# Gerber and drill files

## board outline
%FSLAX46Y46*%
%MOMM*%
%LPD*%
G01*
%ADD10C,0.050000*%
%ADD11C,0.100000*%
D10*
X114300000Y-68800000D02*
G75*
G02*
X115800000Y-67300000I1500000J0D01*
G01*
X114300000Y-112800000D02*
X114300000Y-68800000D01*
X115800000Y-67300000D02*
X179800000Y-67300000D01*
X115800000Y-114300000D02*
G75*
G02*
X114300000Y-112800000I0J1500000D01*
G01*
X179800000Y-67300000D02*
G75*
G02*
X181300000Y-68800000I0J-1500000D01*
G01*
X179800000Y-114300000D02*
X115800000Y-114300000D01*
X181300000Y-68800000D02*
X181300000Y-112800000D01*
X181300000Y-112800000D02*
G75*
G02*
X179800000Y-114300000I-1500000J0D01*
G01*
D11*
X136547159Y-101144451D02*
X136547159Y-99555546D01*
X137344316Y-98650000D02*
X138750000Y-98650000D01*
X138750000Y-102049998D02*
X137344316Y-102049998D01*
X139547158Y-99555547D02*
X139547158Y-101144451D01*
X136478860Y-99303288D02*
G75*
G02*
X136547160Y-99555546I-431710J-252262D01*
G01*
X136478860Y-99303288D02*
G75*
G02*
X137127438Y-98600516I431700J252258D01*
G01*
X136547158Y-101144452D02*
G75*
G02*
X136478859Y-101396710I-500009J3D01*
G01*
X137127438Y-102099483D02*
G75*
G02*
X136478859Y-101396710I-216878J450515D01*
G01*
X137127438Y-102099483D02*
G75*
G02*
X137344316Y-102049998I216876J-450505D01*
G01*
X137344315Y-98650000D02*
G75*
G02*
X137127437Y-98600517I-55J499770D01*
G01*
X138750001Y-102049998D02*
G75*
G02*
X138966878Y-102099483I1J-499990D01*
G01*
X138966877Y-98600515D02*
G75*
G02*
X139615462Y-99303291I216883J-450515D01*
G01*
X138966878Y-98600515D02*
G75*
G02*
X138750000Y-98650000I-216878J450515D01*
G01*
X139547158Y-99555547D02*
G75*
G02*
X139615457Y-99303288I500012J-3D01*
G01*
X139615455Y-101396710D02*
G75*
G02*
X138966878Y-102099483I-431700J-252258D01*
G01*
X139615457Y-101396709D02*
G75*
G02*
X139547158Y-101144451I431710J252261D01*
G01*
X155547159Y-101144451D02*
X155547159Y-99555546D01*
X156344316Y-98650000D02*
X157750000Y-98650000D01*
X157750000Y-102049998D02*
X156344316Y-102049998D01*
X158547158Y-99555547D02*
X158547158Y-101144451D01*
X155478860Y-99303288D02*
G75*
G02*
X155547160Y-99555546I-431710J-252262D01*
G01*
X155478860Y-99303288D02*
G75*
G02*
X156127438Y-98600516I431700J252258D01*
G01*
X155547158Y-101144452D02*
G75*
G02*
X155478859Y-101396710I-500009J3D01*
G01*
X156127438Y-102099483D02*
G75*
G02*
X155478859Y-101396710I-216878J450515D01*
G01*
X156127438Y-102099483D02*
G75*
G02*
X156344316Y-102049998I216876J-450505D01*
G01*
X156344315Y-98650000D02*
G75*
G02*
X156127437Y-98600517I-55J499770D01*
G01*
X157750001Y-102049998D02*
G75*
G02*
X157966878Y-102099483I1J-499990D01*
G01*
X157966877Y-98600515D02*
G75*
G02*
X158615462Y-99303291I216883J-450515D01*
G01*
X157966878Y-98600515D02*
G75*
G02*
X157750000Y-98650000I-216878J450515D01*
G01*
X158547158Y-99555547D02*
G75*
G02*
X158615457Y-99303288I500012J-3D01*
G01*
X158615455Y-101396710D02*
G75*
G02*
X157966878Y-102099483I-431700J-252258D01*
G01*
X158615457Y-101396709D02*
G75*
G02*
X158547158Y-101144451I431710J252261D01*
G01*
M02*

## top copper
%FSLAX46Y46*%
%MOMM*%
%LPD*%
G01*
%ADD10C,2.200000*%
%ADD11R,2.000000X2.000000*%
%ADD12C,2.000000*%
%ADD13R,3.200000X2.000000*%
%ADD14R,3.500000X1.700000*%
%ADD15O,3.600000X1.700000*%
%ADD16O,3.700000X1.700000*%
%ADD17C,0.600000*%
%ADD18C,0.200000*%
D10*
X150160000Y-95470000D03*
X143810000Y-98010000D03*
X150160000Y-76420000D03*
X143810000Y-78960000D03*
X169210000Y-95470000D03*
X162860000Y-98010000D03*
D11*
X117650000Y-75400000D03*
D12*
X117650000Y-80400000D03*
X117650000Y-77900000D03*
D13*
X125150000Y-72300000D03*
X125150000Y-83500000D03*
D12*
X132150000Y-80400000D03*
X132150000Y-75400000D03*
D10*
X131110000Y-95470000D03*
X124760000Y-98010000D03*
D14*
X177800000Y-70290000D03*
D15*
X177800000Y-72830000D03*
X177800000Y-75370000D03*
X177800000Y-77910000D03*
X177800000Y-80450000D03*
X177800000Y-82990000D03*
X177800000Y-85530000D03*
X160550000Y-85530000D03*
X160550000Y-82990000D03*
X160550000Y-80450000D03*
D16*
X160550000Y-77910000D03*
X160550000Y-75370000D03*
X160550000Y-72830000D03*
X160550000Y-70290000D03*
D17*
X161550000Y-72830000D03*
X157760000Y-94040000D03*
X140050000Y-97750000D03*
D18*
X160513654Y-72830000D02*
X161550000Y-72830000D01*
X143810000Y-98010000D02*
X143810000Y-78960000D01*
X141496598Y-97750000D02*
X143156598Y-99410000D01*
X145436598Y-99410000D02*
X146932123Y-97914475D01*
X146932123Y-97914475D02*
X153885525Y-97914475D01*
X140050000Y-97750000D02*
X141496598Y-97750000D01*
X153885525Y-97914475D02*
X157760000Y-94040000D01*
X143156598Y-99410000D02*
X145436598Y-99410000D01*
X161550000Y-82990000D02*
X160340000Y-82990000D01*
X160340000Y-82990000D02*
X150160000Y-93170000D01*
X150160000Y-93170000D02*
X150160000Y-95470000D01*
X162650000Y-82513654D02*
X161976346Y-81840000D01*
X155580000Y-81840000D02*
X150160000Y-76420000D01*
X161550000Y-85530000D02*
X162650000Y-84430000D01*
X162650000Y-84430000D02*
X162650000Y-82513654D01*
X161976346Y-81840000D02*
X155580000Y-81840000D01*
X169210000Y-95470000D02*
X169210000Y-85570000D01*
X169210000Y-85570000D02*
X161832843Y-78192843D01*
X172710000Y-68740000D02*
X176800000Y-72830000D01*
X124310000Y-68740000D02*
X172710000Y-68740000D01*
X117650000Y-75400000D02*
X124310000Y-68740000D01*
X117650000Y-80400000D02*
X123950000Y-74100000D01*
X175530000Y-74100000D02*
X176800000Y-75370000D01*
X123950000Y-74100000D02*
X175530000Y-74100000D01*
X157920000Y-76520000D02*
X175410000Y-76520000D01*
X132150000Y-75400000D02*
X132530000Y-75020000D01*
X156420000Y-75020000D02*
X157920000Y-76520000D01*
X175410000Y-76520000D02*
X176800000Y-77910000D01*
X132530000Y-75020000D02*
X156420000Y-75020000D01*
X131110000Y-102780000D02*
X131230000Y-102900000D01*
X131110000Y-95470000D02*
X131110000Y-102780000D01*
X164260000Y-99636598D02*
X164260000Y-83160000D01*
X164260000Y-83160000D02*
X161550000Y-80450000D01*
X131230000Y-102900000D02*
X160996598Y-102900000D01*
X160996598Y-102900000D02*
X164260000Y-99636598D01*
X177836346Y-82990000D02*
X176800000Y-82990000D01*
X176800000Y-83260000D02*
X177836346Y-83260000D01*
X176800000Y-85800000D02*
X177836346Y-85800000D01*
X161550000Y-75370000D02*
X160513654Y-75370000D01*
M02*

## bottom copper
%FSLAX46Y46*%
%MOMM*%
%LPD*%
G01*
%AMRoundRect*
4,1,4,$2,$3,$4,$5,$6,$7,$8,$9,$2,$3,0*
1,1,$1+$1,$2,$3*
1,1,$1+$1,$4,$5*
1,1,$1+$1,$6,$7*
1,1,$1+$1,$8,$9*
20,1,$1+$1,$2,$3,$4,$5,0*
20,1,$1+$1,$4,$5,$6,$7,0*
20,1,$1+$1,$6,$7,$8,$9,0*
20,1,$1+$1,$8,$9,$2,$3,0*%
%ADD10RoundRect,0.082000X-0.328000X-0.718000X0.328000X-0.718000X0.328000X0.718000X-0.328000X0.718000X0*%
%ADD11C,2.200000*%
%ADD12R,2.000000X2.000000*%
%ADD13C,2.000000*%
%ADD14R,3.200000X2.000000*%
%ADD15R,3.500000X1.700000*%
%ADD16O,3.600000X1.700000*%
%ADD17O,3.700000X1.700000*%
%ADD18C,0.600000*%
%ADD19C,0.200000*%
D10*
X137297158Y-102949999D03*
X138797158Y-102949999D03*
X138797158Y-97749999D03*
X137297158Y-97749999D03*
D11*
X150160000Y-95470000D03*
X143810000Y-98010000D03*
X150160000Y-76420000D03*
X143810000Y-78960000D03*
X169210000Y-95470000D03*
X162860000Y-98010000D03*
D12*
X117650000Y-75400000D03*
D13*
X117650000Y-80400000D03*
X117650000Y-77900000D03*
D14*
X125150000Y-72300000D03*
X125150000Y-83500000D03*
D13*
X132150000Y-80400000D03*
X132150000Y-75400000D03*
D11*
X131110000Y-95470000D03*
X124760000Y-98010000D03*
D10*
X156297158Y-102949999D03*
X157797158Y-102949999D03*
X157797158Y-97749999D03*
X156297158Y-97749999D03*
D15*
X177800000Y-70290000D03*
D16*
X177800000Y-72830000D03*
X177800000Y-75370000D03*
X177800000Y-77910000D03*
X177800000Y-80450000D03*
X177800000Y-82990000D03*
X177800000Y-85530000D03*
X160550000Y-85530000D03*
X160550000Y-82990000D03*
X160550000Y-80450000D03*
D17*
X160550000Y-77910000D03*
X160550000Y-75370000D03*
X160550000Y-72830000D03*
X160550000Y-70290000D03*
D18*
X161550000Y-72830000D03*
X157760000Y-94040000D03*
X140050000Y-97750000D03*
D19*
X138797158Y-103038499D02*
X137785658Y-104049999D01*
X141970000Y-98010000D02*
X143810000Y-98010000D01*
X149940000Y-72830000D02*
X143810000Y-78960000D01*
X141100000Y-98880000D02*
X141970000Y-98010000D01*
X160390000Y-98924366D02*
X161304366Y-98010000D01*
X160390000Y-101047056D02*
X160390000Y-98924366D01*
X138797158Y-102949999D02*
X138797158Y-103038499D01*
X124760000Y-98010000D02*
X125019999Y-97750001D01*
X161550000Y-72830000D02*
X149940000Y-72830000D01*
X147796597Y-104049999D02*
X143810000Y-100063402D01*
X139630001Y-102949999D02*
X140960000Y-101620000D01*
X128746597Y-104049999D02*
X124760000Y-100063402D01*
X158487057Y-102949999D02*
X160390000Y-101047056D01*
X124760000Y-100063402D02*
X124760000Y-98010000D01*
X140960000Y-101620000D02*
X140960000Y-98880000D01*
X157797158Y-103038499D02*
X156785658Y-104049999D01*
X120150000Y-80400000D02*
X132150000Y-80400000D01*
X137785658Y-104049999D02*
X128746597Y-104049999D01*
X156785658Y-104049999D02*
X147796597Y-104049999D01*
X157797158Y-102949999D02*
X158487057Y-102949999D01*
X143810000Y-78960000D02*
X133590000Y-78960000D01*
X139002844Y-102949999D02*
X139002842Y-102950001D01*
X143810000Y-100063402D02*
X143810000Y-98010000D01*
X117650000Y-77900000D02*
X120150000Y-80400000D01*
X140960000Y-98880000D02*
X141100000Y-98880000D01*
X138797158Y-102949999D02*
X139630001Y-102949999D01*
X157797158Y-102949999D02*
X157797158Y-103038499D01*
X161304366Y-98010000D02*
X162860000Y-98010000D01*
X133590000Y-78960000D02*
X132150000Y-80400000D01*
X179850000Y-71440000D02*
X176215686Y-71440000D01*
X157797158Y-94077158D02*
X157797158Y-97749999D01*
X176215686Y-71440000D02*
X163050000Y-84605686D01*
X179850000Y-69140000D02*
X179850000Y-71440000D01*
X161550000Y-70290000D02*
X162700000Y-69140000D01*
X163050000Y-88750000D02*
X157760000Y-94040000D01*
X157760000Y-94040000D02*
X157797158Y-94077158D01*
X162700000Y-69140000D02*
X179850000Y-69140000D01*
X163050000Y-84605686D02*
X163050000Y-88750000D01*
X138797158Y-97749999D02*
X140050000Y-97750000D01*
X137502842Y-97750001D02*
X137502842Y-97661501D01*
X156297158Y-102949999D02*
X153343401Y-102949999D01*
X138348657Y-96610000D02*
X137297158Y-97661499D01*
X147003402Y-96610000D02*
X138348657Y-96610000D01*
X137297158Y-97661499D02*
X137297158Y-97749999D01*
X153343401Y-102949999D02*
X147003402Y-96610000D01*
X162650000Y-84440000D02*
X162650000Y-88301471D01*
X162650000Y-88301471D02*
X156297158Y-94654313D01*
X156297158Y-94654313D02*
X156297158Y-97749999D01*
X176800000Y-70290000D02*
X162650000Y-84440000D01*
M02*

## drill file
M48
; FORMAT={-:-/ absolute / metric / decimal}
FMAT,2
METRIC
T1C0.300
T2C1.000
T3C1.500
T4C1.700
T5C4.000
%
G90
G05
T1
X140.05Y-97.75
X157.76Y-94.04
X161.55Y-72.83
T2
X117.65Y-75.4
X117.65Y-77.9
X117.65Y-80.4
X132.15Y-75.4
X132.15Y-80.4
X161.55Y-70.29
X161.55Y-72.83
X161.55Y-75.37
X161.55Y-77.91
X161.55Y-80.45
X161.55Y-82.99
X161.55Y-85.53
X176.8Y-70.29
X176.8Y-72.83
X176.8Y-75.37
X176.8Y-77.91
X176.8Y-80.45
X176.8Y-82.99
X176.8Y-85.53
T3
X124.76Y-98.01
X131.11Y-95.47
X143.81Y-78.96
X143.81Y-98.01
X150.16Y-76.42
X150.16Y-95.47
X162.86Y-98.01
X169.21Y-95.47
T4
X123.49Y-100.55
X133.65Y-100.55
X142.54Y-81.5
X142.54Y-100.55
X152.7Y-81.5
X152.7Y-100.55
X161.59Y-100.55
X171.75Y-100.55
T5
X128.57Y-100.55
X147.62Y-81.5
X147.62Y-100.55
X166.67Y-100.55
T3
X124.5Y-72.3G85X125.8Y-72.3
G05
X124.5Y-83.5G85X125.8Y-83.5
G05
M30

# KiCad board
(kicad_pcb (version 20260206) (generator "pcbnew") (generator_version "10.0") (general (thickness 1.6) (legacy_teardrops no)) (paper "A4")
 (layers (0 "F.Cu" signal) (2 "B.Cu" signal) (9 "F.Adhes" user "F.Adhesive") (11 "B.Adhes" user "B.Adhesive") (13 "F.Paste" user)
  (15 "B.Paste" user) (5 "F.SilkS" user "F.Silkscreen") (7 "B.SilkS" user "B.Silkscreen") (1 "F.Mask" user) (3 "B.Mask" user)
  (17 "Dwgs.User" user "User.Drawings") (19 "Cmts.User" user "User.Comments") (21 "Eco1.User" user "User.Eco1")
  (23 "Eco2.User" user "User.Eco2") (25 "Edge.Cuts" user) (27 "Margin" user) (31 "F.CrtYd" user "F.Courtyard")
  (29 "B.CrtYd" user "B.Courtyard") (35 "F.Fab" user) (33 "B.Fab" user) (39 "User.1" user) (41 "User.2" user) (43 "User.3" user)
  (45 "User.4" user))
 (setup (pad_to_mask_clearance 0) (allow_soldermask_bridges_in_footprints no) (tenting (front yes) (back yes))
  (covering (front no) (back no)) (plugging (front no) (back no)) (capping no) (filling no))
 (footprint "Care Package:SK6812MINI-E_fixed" (layer "F.Cu") (at 138.15 100.35 90)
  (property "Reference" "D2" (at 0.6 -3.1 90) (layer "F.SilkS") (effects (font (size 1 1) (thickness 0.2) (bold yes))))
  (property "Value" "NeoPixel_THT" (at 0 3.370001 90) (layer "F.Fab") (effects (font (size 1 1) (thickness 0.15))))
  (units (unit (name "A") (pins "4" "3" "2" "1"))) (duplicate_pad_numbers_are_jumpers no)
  (fp_line (start -0.794451 -1.602841) (end 0.794454 -1.602841) (stroke (width 0.1) (type solid)) (layer "Edge.Cuts"))
  (fp_line (start 1.7 -0.805684) (end 1.7 0.6) (stroke (width 0.1) (type solid)) (layer "Edge.Cuts"))
  (fp_line (start -1.699998 0.6) (end -1.699998 -0.805684) (stroke (width 0.1) (type solid)) (layer "Edge.Cuts"))
  (fp_line (start 0.794453 1.397158) (end -0.794451 1.397158) (stroke (width 0.1) (type solid)) (layer "Edge.Cuts"))
  (fp_arc (start 1.046712 -1.67114) (mid 0.925124 -1.620218) (end 0.794454 -1.602841) (stroke (width 0.1) (type solid)) (layer "Edge.Cuts"))
  (fp_arc (start 1.046712 -1.67114) (mid 1.638071 -1.606876) (end 1.749485 -1.022562) (stroke (width 0.1) (type solid)) (layer "Edge.Cuts"))
  (fp_arc (start -0.794452 -1.602842) (mid -0.925122 -1.620219) (end -1.04671 -1.671141) (stroke (width 0.1) (type solid))
   (layer "Edge.Cuts"))
  (fp_arc (start -1.749483 -1.022562) (mid -1.63807 -1.606877) (end -1.04671 -1.671141) (stroke (width 0.1) (type solid))
   (layer "Edge.Cuts"))
  (fp_arc (start -1.749483 -1.022562) (mid -1.712526 -0.91691) (end -1.699998 -0.805684) (stroke (width 0.1) (type solid))
   (layer "Edge.Cuts"))
  (fp_arc (start 1.7 -0.805685) (mid 1.712523 -0.916913) (end 1.749485 -1.022562) (stroke (width 0.1) (type solid)) (layer "Edge.Cuts"))
  (fp_arc (start -1.699998 0.600001) (mid -1.712526 0.711226) (end -1.749483 0.816878) (stroke (width 0.1) (type solid)) (layer "Edge.Cuts"))
  (fp_arc (start 1.749485 0.816877) (mid 1.638074 1.401197) (end 1.046712 1.465457) (stroke (width 0.1) (type solid)) (layer "Edge.Cuts"))
  (fp_arc (start 1.749485 0.816878) (mid 1.712528 0.711226) (end 1.7 0.6) (stroke (width 0.1) (type solid)) (layer "Edge.Cuts"))
  (fp_arc (start 0.794453 1.397158) (mid 0.925124 1.414535) (end 1.046712 1.465457) (stroke (width 0.1) (type solid)) (layer "Edge.Cuts"))
  (fp_arc (start -1.04671 1.465455) (mid -1.638069 1.401192) (end -1.749483 0.816878) (stroke (width 0.1) (type solid)) (layer "Edge.Cuts"))
  (fp_arc (start -1.046709 1.465457) (mid -0.925121 1.414535) (end -0.794451 1.397158) (stroke (width 0.1) (type solid)) (layer "Edge.Cuts"))
  (pad "1" smd roundrect (at -2.599999 -0.852842) (size 0.82 1.6) (layers "B.Cu" "B.Mask" "B.Paste") (roundrect_rratio 0.1)
   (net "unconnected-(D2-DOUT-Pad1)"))
  (pad "2" smd roundrect (at -2.599999 0.647158) (size 0.82 1.6) (layers "B.Cu" "B.Mask" "B.Paste") (roundrect_rratio 0.1) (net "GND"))
  (pad "3" smd roundrect (at 2.600001 0.647158) (size 0.82 1.6) (layers "B.Cu" "B.Mask" "B.Paste") (roundrect_rratio 0.1) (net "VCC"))
  (pad "4" smd roundrect (at 2.600001 -0.852842) (size 0.82 1.6) (layers "B.Cu" "B.Mask" "B.Paste") (roundrect_rratio 0.1)
   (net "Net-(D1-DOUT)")))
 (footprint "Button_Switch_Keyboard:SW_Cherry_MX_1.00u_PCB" (layer "F.Cu") (at 150.16 95.47)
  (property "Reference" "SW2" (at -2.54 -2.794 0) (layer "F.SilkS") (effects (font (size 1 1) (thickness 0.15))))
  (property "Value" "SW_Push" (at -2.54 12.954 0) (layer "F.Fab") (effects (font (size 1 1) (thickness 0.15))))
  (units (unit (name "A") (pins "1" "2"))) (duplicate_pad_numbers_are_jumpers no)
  (pad "" np_thru_hole circle (at -7.62 5.08) (size 1.7 1.7) (drill 1.7) (layers "*.Cu" "*.Mask"))
  (pad "" np_thru_hole circle (at -2.54 5.08) (size 4 4) (drill 4) (layers "*.Cu" "*.Mask"))
  (pad "" np_thru_hole circle (at 2.54 5.08) (size 1.7 1.7) (drill 1.7) (layers "*.Cu" "*.Mask"))
  (pad "1" thru_hole circle (at 0 0) (size 2.2 2.2) (drill 1.5) (layers "*.Cu" "*.Mask") (remove_unused_layers no)
   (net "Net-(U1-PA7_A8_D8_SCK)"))
  (pad "2" thru_hole circle (at -6.35 2.54) (size 2.2 2.2) (drill 1.5) (layers "*.Cu" "*.Mask") (remove_unused_layers no) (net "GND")))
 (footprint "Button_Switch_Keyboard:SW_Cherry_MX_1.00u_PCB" (layer "F.Cu") (at 150.16 76.42)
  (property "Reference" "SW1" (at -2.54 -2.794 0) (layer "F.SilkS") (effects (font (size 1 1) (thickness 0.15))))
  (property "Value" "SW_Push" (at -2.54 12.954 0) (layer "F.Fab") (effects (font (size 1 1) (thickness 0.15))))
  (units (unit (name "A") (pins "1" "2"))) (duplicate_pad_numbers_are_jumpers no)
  (pad "" np_thru_hole circle (at -7.62 5.08) (size 1.7 1.7) (drill 1.7) (layers "*.Cu" "*.Mask"))
  (pad "" np_thru_hole circle (at -2.54 5.08) (size 4 4) (drill 4) (layers "*.Cu" "*.Mask"))
  (pad "" np_thru_hole circle (at 2.54 5.08) (size 1.7 1.7) (drill 1.7) (layers "*.Cu" "*.Mask"))
  (pad "1" thru_hole circle (at 0 0) (size 2.2 2.2) (drill 1.5) (layers "*.Cu" "*.Mask") (remove_unused_layers no)
   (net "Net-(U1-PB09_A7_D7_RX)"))
  (pad "2" thru_hole circle (at -6.35 2.54) (size 2.2 2.2) (drill 1.5) (layers "*.Cu" "*.Mask") (remove_unused_layers no) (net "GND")))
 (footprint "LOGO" (layer "F.Cu") (at 176.41 109.06)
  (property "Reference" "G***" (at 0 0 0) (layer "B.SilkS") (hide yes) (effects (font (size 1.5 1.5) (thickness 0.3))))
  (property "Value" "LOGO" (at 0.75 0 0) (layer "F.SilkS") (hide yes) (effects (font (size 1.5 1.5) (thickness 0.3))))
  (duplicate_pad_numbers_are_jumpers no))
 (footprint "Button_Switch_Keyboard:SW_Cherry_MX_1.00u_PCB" (layer "F.Cu") (at 169.21 95.47)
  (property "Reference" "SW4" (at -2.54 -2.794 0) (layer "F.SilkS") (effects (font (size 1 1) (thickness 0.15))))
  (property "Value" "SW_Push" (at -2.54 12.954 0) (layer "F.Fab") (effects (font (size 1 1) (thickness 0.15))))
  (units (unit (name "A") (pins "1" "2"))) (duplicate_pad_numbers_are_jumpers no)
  (pad "" np_thru_hole circle (at -7.62 5.08) (size 1.7 1.7) (drill 1.7) (layers "*.Cu" "*.Mask"))
  (pad "" np_thru_hole circle (at -2.54 5.08) (size 4 4) (drill 4) (layers "*.Cu" "*.Mask"))
  (pad "" np_thru_hole circle (at 2.54 5.08) (size 1.7 1.7) (drill 1.7) (layers "*.Cu" "*.Mask"))
  (pad "1" thru_hole circle (at 0 0) (size 2.2 2.2) (drill 1.5) (layers "*.Cu" "*.Mask") (remove_unused_layers no)
   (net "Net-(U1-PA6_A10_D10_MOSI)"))
  (pad "2" thru_hole circle (at -6.35 2.54) (size 2.2 2.2) (drill 1.5) (layers "*.Cu" "*.Mask") (remove_unused_layers no) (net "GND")))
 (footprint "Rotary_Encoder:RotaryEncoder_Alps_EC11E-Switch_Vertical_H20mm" (layer "F.Cu") (at 117.65 75.4)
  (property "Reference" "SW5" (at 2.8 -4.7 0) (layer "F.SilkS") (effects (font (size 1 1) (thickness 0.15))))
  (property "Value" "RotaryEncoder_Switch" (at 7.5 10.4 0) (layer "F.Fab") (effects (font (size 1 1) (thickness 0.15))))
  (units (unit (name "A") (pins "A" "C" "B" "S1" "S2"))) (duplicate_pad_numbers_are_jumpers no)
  (pad "A" thru_hole rect (at 0 0) (size 2 2) (drill 1) (layers "*.Cu" "*.Mask") (remove_unused_layers no) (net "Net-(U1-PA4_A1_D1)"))
  (pad "B" thru_hole circle (at 0 5) (size 2 2) (drill 1) (layers "*.Cu" "*.Mask") (remove_unused_layers no) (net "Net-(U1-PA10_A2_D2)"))
  (pad "C" thru_hole circle (at 0 2.5) (size 2 2) (drill 1) (layers "*.Cu" "*.Mask") (remove_unused_layers no) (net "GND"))
  (pad "MP" thru_hole rect (at 7.5 -3.1) (size 3.2 2) (drill oval 2.8 1.5) (layers "*.Cu" "*.Mask") (remove_unused_layers no))
  (pad "MP" thru_hole rect (at 7.5 8.1) (size 3.2 2) (drill oval 2.8 1.5) (layers "*.Cu" "*.Mask") (remove_unused_layers no))
  (pad "S1" thru_hole circle (at 14.5 5) (size 2 2) (drill 1) (layers "*.Cu" "*.Mask") (remove_unused_layers no) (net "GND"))
  (pad "S2" thru_hole circle (at 14.5 0) (size 2 2) (drill 1) (layers "*.Cu" "*.Mask") (remove_unused_layers no) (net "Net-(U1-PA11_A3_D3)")))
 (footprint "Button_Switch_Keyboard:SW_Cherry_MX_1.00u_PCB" (layer "F.Cu") (at 131.11 95.47)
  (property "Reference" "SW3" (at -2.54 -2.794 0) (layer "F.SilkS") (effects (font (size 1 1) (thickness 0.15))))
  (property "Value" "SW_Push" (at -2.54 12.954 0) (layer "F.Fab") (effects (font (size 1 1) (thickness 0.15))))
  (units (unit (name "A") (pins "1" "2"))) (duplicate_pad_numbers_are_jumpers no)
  (pad "" np_thru_hole circle (at -7.62 5.08) (size 1.7 1.7) (drill 1.7) (layers "*.Cu" "*.Mask"))
  (pad "" np_thru_hole circle (at -2.54 5.08) (size 4 4) (drill 4) (layers "*.Cu" "*.Mask"))
  (pad "" np_thru_hole circle (at 2.54 5.08) (size 1.7 1.7) (drill 1.7) (layers "*.Cu" "*.Mask"))
  (pad "1" thru_hole circle (at 0 0) (size 2.2 2.2) (drill 1.5) (layers "*.Cu" "*.Mask") (remove_unused_layers no)
   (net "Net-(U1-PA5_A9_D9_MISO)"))
  (pad "2" thru_hole circle (at -6.35 2.54) (size 2.2 2.2) (drill 1.5) (layers "*.Cu" "*.Mask") (remove_unused_layers no) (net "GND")))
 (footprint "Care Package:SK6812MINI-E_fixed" (layer "F.Cu") (at 157.15 100.35 90)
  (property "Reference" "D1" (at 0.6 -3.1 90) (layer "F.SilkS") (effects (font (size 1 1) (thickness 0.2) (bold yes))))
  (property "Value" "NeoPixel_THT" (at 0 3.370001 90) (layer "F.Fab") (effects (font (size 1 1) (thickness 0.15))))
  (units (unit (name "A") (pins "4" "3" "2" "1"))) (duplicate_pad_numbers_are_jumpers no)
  (fp_line (start -0.794451 -1.602841) (end 0.794454 -1.602841) (stroke (width 0.1) (type solid)) (layer "Edge.Cuts"))
  (fp_line (start 1.7 -0.805684) (end 1.7 0.6) (stroke (width 0.1) (type solid)) (layer "Edge.Cuts"))
  (fp_line (start -1.699998 0.6) (end -1.699998 -0.805684) (stroke (width 0.1) (type solid)) (layer "Edge.Cuts"))
  (fp_line (start 0.794453 1.397158) (end -0.794451 1.397158) (stroke (width 0.1) (type solid)) (layer "Edge.Cuts"))
  (fp_arc (start 1.046712 -1.67114) (mid 0.925124 -1.620218) (end 0.794454 -1.602841) (stroke (width 0.1) (type solid)) (layer "Edge.Cuts"))
  (fp_arc (start 1.046712 -1.67114) (mid 1.638071 -1.606876) (end 1.749485 -1.022562) (stroke (width 0.1) (type solid)) (layer "Edge.Cuts"))
  (fp_arc (start -0.794452 -1.602842) (mid -0.925122 -1.620219) (end -1.04671 -1.671141) (stroke (width 0.1) (type solid))
   (layer "Edge.Cuts"))
  (fp_arc (start -1.749483 -1.022562) (mid -1.63807 -1.606877) (end -1.04671 -1.671141) (stroke (width 0.1) (type solid))
   (layer "Edge.Cuts"))
  (fp_arc (start -1.749483 -1.022562) (mid -1.712526 -0.91691) (end -1.699998 -0.805684) (stroke (width 0.1) (type solid))
   (layer "Edge.Cuts"))
  (fp_arc (start 1.7 -0.805685) (mid 1.712523 -0.916913) (end 1.749485 -1.022562) (stroke (width 0.1) (type solid)) (layer "Edge.Cuts"))
  (fp_arc (start -1.699998 0.600001) (mid -1.712526 0.711226) (end -1.749483 0.816878) (stroke (width 0.1) (type solid)) (layer "Edge.Cuts"))
  (fp_arc (start 1.749485 0.816877) (mid 1.638074 1.401197) (end 1.046712 1.465457) (stroke (width 0.1) (type solid)) (layer "Edge.Cuts"))
  (fp_arc (start 1.749485 0.816878) (mid 1.712528 0.711226) (end 1.7 0.6) (stroke (width 0.1) (type solid)) (layer "Edge.Cuts"))
  (fp_arc (start 0.794453 1.397158) (mid 0.925124 1.414535) (end 1.046712 1.465457) (stroke (width 0.1) (type solid)) (layer "Edge.Cuts"))
  (fp_arc (start -1.04671 1.465455) (mid -1.638069 1.401192) (end -1.749483 0.816878) (stroke (width 0.1) (type solid)) (layer "Edge.Cuts"))
  (fp_arc (start -1.046709 1.465457) (mid -0.925121 1.414535) (end -0.794451 1.397158) (stroke (width 0.1) (type solid)) (layer "Edge.Cuts"))
  (pad "1" smd roundrect (at -2.599999 -0.852842) (size 0.82 1.6) (layers "B.Cu" "B.Mask" "B.Paste") (roundrect_rratio 0.1)
   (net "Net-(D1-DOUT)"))
  (pad "2" smd roundrect (at -2.599999 0.647158) (size 0.82 1.6) (layers "B.Cu" "B.Mask" "B.Paste") (roundrect_rratio 0.1) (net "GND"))
  (pad "3" smd roundrect (at 2.600001 0.647158) (size 0.82 1.6) (layers "B.Cu" "B.Mask" "B.Paste") (roundrect_rratio 0.1) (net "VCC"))
  (pad "4" smd roundrect (at 2.600001 -0.852842) (size 0.82 1.6) (layers "B.Cu" "B.Mask" "B.Paste") (roundrect_rratio 0.1)
   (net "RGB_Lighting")))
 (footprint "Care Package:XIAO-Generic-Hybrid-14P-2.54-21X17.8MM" (layer "B.Cu") (at 169.175 77.91 180)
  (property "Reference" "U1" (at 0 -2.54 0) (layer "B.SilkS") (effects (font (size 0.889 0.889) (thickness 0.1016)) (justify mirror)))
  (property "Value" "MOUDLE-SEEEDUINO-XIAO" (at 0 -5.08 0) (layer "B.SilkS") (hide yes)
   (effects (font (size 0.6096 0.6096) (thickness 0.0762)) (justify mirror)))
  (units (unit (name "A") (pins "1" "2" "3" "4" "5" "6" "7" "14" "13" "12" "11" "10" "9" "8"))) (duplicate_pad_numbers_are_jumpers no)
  (pad "1" thru_hole rect (at -7.625 7.62 180) (size 3.5 1.7) (drill 1 (offset -1 0)) (layers "*.Cu" "*.Mask") (remove_unused_layers no)
   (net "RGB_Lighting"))
  (pad "2" thru_hole oval (at -7.625 5.08 180) (size 3.6 1.7) (drill 1 (offset -1 0)) (layers "*.Cu" "*.Mask") (remove_unused_layers no)
   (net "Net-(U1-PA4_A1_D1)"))
  (pad "3" thru_hole oval (at -7.625 2.54 180) (size 3.6 1.7) (drill 1 (offset -1 0)) (layers "*.Cu" "*.Mask") (remove_unused_layers no)
   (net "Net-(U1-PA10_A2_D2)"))
  (pad "4" thru_hole oval (at -7.625 0 180) (size 3.6 1.7) (drill 1 (offset -1 0)) (layers "*.Cu" "*.Mask") (remove_unused_layers no)
   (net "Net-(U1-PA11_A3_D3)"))
  (pad "5" thru_hole oval (at -7.625 -2.54 180) (size 3.6 1.7) (drill 1 (offset -1 0)) (layers "*.Cu" "*.Mask") (remove_unused_layers no)
   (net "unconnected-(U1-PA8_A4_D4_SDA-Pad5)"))
  (pad "6" thru_hole oval (at -7.625 -5.08) (size 3.6 1.7) (drill 1 (offset 1 0)) (layers "*.Cu" "*.Mask") (remove_unused_layers no)
   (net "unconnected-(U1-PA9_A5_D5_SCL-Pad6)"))
  (pad "7" thru_hole oval (at -7.625 -7.62 180) (size 3.6 1.7) (drill 1 (offset -1 0)) (layers "*.Cu" "*.Mask") (remove_unused_layers no)
   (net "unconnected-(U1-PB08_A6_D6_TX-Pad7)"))
  (pad "8" thru_hole oval (at 7.625 -7.62 180) (size 3.6 1.7) (drill 1 (offset 1 0)) (layers "*.Cu" "*.Mask") (remove_unused_layers no)
   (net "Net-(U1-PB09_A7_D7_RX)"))
  (pad "9" thru_hole oval (at 7.625 -5.08 180) (size 3.6 1.7) (drill 1 (offset 1 0)) (layers "*.Cu" "*.Mask") (remove_unused_layers no)
   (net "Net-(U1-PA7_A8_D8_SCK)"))
  (pad "10" thru_hole oval (at 7.625 -2.54 180) (size 3.6 1.7) (drill 1 (offset 1 0)) (layers "*.Cu" "*.Mask") (remove_unused_layers no)
   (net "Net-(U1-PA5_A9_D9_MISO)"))
  (pad "11" thru_hole oval (at 7.625 0 180) (size 3.7 1.7) (drill 1 (offset 1 0)) (layers "*.Cu" "*.Mask") (remove_unused_layers no)
   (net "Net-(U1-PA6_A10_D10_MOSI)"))
  (pad "12" thru_hole oval (at 7.625 2.54 180) (size 3.7 1.7) (drill 1 (offset 1 0)) (layers "*.Cu" "*.Mask") (remove_unused_layers no)
   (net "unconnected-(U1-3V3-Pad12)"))
  (pad "13" thru_hole oval (at 7.625 5.08 180) (size 3.7 1.7) (drill 1 (offset 1 0)) (layers "*.Cu" "*.Mask") (remove_unused_layers no)
   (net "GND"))
  (pad "14" thru_hole oval (at 7.625 7.62 180) (size 3.7 1.7) (drill 1 (offset 1 0)) (layers "*.Cu" "*.Mask") (remove_unused_layers no)
   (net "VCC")))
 (gr_arc (start 114.3 68.8) (mid 114.73934 67.73934) (end 115.8 67.3) (stroke (width 0.05) (type default)) (layer "Edge.Cuts"))
 (gr_line (start 114.3 112.8) (end 114.3 68.8) (stroke (width 0.05) (type default)) (layer "Edge.Cuts"))
 (gr_line (start 115.8 67.3) (end 179.8 67.3) (stroke (width 0.05) (type default)) (layer "Edge.Cuts"))
 (gr_arc (start 115.8 114.3) (mid 114.73934 113.86066) (end 114.3 112.8) (stroke (width 0.05) (type default)) (layer "Edge.Cuts"))
 (gr_arc (start 179.8 67.3) (mid 180.86066 67.73934) (end 181.3 68.8) (stroke (width 0.05) (type default)) (layer "Edge.Cuts"))
 (gr_line (start 179.8 114.3) (end 115.8 114.3) (stroke (width 0.05) (type default)) (layer "Edge.Cuts"))
 (gr_line (start 181.3 68.8) (end 181.3 112.8) (stroke (width 0.05) (type default)) (layer "Edge.Cuts"))
 (gr_arc (start 181.3 112.8) (mid 180.86066 113.86066) (end 179.8 114.3) (stroke (width 0.05) (type default)) (layer "Edge.Cuts"))
 (segment (start 160.513654 72.83) (end 161.55 72.83) (width 0.2) (layer "F.Cu") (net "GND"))
 (segment (start 143.81 98.01) (end 143.81 78.96) (width 0.2) (layer "F.Cu") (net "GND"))
 (via (at 161.55 72.83) (size 0.6) (drill 0.3) (layers "F.Cu" "B.Cu") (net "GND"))
 (segment (start 138.797158 103.038499) (end 137.785658 104.049999) (width 0.2) (layer "B.Cu") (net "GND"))
 (segment (start 141.97 98.01) (end 143.81 98.01) (width 0.2) (layer "B.Cu") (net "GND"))
 (segment (start 149.94 72.83) (end 143.81 78.96) (width 0.2) (layer "B.Cu") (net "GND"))
 (segment (start 141.1 98.88) (end 141.97 98.01) (width 0.2) (layer "B.Cu") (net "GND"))
 (segment (start 160.39 98.924366) (end 161.304366 98.01) (width 0.2) (layer "B.Cu") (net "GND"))
 (segment (start 160.39 101.047056) (end 160.39 98.924366) (width 0.2) (layer "B.Cu") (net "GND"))
 (segment (start 138.797158 102.949999) (end 138.797158 103.038499) (width 0.2) (layer "B.Cu") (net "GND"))
 (segment (start 124.76 98.01) (end 125.019999 97.750001) (width 0.2) (layer "B.Cu") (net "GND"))
 (segment (start 161.55 72.83) (end 149.94 72.83) (width 0.2) (layer "B.Cu") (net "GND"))
 (segment (start 147.796597 104.049999) (end 143.81 100.063402) (width 0.2) (layer "B.Cu") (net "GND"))
 (segment (start 139.630001 102.949999) (end 140.96 101.62) (width 0.2) (layer "B.Cu") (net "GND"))
 (segment (start 128.746597 104.049999) (end 124.76 100.063402) (width 0.2) (layer "B.Cu") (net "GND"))
 (segment (start 158.487057 102.949999) (end 160.39 101.047056) (width 0.2) (layer "B.Cu") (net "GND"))
 (segment (start 124.76 100.063402) (end 124.76 98.01) (width 0.2) (layer "B.Cu") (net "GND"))
 (segment (start 140.96 101.62) (end 140.96 98.88) (width 0.2) (layer "B.Cu") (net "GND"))
 (segment (start 157.797158 103.038499) (end 156.785658 104.049999) (width 0.2) (layer "B.Cu") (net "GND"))
 (segment (start 120.15 80.4) (end 132.15 80.4) (width 0.2) (layer "B.Cu") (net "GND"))
 (segment (start 137.785658 104.049999) (end 128.746597 104.049999) (width 0.2) (layer "B.Cu") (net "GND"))
 (segment (start 156.785658 104.049999) (end 147.796597 104.049999) (width 0.2) (layer "B.Cu") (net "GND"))
 (segment (start 157.797158 102.949999) (end 158.487057 102.949999) (width 0.2) (layer "B.Cu") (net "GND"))
 (segment (start 143.81 78.96) (end 133.59 78.96) (width 0.2) (layer "B.Cu") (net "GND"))
 (segment (start 139.002844 102.949999) (end 139.002842 102.950001) (width 0.2) (layer "B.Cu") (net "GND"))
 (segment (start 143.81 100.063402) (end 143.81 98.01) (width 0.2) (layer "B.Cu") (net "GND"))
 (segment (start 117.65 77.9) (end 120.15 80.4) (width 0.2) (layer "B.Cu") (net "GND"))
 (segment (start 140.96 98.88) (end 141.1 98.88) (width 0.2) (layer "B.Cu") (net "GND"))
 (segment (start 138.797158 102.949999) (end 139.630001 102.949999) (width 0.2) (layer "B.Cu") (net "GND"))
 (segment (start 157.797158 102.949999) (end 157.797158 103.038499) (width 0.2) (layer "B.Cu") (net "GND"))
 (segment (start 161.304366 98.01) (end 162.86 98.01) (width 0.2) (layer "B.Cu") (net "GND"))
 (segment (start 133.59 78.96) (end 132.15 80.4) (width 0.2) (layer "B.Cu") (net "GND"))
 (segment (start 141.496598 97.75) (end 143.156598 99.41) (width 0.2) (layer "F.Cu") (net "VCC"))
 (segment (start 145.436598 99.41) (end 146.932123 97.914475) (width 0.2) (layer "F.Cu") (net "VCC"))
 (segment (start 146.932123 97.914475) (end 153.885525 97.914475) (width 0.2) (layer "F.Cu") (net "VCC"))
 (segment (start 140.05 97.75) (end 141.496598 97.75) (width 0.2) (layer "F.Cu") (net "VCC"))
 (segment (start 153.885525 97.914475) (end 157.76 94.04) (width 0.2) (layer "F.Cu") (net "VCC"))
 (segment (start 143.156598 99.41) (end 145.436598 99.41) (width 0.2) (layer "F.Cu") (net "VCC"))
 (via (at 157.76 94.04) (size 0.6) (drill 0.3) (layers "F.Cu" "B.Cu") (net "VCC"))
 (via (at 140.05 97.75) (size 0.6) (drill 0.3) (layers "F.Cu" "B.Cu") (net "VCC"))
 (segment (start 179.85 71.44) (end 176.215686 71.44) (width 0.2) (layer "B.Cu") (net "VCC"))
 (segment (start 157.797158 94.077158) (end 157.797158 97.749999) (width 0.2) (layer "B.Cu") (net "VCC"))
 (segment (start 176.215686 71.44) (end 163.05 84.605686) (width 0.2) (layer "B.Cu") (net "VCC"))
 (segment (start 179.85 69.14) (end 179.85 71.44) (width 0.2) (layer "B.Cu") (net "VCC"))
 (segment (start 161.55 70.29) (end 162.7 69.14) (width 0.2) (layer "B.Cu") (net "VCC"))
 (segment (start 163.05 88.75) (end 157.76 94.04) (width 0.2) (layer "B.Cu") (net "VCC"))
 (segment (start 157.76 94.04) (end 157.797158 94.077158) (width 0.2) (layer "B.Cu") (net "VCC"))
 (segment (start 162.7 69.14) (end 179.85 69.14) (width 0.2) (layer "B.Cu") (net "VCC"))
 (segment (start 163.05 84.605686) (end 163.05 88.75) (width 0.2) (layer "B.Cu") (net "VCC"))
 (segment (start 138.797158 97.749999) (end 140.05 97.75) (width 0.2) (layer "B.Cu") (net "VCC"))
 (segment (start 137.502842 97.750001) (end 137.502842 97.661501) (width 0.2) (layer "B.Cu") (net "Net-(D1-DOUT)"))
 (segment (start 156.297158 102.949999) (end 153.343401 102.949999) (width 0.2) (layer "B.Cu") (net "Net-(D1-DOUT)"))
 (segment (start 138.348657 96.61) (end 137.297158 97.661499) (width 0.2) (layer "B.Cu") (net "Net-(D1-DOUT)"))
 (segment (start 147.003402 96.61) (end 138.348657 96.61) (width 0.2) (layer "B.Cu") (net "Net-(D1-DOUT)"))
 (segment (start 137.297158 97.661499) (end 137.297158 97.749999) (width 0.2) (layer "B.Cu") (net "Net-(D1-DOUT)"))
 (segment (start 153.343401 102.949999) (end 147.003402 96.61) (width 0.2) (layer "B.Cu") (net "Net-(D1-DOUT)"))
 (segment (start 161.55 82.99) (end 160.34 82.99) (width 0.2) (layer "F.Cu") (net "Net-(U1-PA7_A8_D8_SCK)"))
 (segment (start 160.34 82.99) (end 150.16 93.17) (width 0.2) (layer "F.Cu") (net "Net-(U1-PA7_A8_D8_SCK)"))
 (segment (start 150.16 93.17) (end 150.16 95.47) (width 0.2) (layer "F.Cu") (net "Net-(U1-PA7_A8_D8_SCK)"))
 (segment (start 162.65 82.513654) (end 161.976346 81.84) (width 0.2) (layer "F.Cu") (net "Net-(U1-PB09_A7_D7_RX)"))
 (segment (start 155.58 81.84) (end 150.16 76.42) (width 0.2) (layer "F.Cu") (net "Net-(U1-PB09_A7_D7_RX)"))
 (segment (start 161.55 85.53) (end 162.65 84.43) (width 0.2) (layer "F.Cu") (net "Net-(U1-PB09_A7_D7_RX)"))
 (segment (start 162.65 84.43) (end 162.65 82.513654) (width 0.2) (layer "F.Cu") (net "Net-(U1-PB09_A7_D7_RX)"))
 (segment (start 161.976346 81.84) (end 155.58 81.84) (width 0.2) (layer "F.Cu") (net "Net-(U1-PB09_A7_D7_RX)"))
 (segment (start 169.21 95.47) (end 169.21 85.57) (width 0.2) (layer "F.Cu") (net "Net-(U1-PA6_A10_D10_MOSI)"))
 (segment (start 169.21 85.57) (end 161.832843 78.192843) (width 0.2) (layer "F.Cu") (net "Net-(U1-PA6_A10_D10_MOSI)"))
 (segment (start 172.71 68.74) (end 176.8 72.83) (width 0.2) (layer "F.Cu") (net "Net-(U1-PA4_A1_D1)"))
 (segment (start 124.31 68.74) (end 172.71 68.74) (width 0.2) (layer "F.Cu") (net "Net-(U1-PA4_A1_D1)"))
 (segment (start 117.65 75.4) (end 124.31 68.74) (width 0.2) (layer "F.Cu") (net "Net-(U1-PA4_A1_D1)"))
 (segment (start 117.65 80.4) (end 123.95 74.1) (width 0.2) (layer "F.Cu") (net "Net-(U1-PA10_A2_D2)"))
 (segment (start 175.53 74.1) (end 176.8 75.37) (width 0.2) (layer "F.Cu") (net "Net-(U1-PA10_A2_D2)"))
 (segment (start 123.95 74.1) (end 175.53 74.1) (width 0.2) (layer "F.Cu") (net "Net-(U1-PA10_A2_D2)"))
 (segment (start 157.92 76.52) (end 175.41 76.52) (width 0.2) (layer "F.Cu") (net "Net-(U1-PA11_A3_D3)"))
 (segment (start 132.15 75.4) (end 132.53 75.02) (width 0.2) (layer "F.Cu") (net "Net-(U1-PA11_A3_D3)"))
 (segment (start 156.42 75.02) (end 157.92 76.52) (width 0.2) (layer "F.Cu") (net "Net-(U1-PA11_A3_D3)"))
 (segment (start 175.41 76.52) (end 176.8 77.91) (width 0.2) (layer "F.Cu") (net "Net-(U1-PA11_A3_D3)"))
 (segment (start 132.53 75.02) (end 156.42 75.02) (width 0.2) (layer "F.Cu") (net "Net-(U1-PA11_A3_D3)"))
 (segment (start 131.11 102.78) (end 131.23 102.9) (width 0.2) (layer "F.Cu") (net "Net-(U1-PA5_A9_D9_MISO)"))
 (segment (start 131.11 95.47) (end 131.11 102.78) (width 0.2) (layer "F.Cu") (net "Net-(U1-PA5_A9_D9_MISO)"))
 (segment (start 164.26 99.636598) (end 164.26 83.16) (width 0.2) (layer "F.Cu") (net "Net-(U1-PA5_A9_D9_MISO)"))
 (segment (start 164.26 83.16) (end 161.55 80.45) (width 0.2) (layer "F.Cu") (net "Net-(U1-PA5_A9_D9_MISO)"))
 (segment (start 131.23 102.9) (end 160.996598 102.9) (width 0.2) (layer "F.Cu") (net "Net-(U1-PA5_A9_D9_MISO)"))
 (segment (start 160.996598 102.9) (end 164.26 99.636598) (width 0.2) (layer "F.Cu") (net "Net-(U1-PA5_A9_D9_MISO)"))
 (segment (start 162.65 84.44) (end 162.65 88.301471) (width 0.2) (layer "B.Cu") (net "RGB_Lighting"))
 (segment (start 162.65 88.301471) (end 156.297158 94.654313) (width 0.2) (layer "B.Cu") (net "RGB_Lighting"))
 (segment (start 156.297158 94.654313) (end 156.297158 97.749999) (width 0.2) (layer "B.Cu") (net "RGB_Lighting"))
 (segment (start 176.8 70.29) (end 162.65 84.44) (width 0.2) (layer "B.Cu") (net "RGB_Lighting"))
 (segment (start 177.836346 82.99) (end 176.8 82.99) (width 0.2) (layer "F.Cu") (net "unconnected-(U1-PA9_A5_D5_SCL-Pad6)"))
 (segment (start 176.8 83.26) (end 177.836346 83.26) (width 0.2) (layer "F.Cu") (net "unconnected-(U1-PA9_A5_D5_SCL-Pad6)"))
 (segment (start 176.8 85.8) (end 177.836346 85.8) (width 0.2) (layer "F.Cu") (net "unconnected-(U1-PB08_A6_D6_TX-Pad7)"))
 (segment (start 161.55 75.37) (end 160.513654 75.37) (width 0.2) (layer "F.Cu") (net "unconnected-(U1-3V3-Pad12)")))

